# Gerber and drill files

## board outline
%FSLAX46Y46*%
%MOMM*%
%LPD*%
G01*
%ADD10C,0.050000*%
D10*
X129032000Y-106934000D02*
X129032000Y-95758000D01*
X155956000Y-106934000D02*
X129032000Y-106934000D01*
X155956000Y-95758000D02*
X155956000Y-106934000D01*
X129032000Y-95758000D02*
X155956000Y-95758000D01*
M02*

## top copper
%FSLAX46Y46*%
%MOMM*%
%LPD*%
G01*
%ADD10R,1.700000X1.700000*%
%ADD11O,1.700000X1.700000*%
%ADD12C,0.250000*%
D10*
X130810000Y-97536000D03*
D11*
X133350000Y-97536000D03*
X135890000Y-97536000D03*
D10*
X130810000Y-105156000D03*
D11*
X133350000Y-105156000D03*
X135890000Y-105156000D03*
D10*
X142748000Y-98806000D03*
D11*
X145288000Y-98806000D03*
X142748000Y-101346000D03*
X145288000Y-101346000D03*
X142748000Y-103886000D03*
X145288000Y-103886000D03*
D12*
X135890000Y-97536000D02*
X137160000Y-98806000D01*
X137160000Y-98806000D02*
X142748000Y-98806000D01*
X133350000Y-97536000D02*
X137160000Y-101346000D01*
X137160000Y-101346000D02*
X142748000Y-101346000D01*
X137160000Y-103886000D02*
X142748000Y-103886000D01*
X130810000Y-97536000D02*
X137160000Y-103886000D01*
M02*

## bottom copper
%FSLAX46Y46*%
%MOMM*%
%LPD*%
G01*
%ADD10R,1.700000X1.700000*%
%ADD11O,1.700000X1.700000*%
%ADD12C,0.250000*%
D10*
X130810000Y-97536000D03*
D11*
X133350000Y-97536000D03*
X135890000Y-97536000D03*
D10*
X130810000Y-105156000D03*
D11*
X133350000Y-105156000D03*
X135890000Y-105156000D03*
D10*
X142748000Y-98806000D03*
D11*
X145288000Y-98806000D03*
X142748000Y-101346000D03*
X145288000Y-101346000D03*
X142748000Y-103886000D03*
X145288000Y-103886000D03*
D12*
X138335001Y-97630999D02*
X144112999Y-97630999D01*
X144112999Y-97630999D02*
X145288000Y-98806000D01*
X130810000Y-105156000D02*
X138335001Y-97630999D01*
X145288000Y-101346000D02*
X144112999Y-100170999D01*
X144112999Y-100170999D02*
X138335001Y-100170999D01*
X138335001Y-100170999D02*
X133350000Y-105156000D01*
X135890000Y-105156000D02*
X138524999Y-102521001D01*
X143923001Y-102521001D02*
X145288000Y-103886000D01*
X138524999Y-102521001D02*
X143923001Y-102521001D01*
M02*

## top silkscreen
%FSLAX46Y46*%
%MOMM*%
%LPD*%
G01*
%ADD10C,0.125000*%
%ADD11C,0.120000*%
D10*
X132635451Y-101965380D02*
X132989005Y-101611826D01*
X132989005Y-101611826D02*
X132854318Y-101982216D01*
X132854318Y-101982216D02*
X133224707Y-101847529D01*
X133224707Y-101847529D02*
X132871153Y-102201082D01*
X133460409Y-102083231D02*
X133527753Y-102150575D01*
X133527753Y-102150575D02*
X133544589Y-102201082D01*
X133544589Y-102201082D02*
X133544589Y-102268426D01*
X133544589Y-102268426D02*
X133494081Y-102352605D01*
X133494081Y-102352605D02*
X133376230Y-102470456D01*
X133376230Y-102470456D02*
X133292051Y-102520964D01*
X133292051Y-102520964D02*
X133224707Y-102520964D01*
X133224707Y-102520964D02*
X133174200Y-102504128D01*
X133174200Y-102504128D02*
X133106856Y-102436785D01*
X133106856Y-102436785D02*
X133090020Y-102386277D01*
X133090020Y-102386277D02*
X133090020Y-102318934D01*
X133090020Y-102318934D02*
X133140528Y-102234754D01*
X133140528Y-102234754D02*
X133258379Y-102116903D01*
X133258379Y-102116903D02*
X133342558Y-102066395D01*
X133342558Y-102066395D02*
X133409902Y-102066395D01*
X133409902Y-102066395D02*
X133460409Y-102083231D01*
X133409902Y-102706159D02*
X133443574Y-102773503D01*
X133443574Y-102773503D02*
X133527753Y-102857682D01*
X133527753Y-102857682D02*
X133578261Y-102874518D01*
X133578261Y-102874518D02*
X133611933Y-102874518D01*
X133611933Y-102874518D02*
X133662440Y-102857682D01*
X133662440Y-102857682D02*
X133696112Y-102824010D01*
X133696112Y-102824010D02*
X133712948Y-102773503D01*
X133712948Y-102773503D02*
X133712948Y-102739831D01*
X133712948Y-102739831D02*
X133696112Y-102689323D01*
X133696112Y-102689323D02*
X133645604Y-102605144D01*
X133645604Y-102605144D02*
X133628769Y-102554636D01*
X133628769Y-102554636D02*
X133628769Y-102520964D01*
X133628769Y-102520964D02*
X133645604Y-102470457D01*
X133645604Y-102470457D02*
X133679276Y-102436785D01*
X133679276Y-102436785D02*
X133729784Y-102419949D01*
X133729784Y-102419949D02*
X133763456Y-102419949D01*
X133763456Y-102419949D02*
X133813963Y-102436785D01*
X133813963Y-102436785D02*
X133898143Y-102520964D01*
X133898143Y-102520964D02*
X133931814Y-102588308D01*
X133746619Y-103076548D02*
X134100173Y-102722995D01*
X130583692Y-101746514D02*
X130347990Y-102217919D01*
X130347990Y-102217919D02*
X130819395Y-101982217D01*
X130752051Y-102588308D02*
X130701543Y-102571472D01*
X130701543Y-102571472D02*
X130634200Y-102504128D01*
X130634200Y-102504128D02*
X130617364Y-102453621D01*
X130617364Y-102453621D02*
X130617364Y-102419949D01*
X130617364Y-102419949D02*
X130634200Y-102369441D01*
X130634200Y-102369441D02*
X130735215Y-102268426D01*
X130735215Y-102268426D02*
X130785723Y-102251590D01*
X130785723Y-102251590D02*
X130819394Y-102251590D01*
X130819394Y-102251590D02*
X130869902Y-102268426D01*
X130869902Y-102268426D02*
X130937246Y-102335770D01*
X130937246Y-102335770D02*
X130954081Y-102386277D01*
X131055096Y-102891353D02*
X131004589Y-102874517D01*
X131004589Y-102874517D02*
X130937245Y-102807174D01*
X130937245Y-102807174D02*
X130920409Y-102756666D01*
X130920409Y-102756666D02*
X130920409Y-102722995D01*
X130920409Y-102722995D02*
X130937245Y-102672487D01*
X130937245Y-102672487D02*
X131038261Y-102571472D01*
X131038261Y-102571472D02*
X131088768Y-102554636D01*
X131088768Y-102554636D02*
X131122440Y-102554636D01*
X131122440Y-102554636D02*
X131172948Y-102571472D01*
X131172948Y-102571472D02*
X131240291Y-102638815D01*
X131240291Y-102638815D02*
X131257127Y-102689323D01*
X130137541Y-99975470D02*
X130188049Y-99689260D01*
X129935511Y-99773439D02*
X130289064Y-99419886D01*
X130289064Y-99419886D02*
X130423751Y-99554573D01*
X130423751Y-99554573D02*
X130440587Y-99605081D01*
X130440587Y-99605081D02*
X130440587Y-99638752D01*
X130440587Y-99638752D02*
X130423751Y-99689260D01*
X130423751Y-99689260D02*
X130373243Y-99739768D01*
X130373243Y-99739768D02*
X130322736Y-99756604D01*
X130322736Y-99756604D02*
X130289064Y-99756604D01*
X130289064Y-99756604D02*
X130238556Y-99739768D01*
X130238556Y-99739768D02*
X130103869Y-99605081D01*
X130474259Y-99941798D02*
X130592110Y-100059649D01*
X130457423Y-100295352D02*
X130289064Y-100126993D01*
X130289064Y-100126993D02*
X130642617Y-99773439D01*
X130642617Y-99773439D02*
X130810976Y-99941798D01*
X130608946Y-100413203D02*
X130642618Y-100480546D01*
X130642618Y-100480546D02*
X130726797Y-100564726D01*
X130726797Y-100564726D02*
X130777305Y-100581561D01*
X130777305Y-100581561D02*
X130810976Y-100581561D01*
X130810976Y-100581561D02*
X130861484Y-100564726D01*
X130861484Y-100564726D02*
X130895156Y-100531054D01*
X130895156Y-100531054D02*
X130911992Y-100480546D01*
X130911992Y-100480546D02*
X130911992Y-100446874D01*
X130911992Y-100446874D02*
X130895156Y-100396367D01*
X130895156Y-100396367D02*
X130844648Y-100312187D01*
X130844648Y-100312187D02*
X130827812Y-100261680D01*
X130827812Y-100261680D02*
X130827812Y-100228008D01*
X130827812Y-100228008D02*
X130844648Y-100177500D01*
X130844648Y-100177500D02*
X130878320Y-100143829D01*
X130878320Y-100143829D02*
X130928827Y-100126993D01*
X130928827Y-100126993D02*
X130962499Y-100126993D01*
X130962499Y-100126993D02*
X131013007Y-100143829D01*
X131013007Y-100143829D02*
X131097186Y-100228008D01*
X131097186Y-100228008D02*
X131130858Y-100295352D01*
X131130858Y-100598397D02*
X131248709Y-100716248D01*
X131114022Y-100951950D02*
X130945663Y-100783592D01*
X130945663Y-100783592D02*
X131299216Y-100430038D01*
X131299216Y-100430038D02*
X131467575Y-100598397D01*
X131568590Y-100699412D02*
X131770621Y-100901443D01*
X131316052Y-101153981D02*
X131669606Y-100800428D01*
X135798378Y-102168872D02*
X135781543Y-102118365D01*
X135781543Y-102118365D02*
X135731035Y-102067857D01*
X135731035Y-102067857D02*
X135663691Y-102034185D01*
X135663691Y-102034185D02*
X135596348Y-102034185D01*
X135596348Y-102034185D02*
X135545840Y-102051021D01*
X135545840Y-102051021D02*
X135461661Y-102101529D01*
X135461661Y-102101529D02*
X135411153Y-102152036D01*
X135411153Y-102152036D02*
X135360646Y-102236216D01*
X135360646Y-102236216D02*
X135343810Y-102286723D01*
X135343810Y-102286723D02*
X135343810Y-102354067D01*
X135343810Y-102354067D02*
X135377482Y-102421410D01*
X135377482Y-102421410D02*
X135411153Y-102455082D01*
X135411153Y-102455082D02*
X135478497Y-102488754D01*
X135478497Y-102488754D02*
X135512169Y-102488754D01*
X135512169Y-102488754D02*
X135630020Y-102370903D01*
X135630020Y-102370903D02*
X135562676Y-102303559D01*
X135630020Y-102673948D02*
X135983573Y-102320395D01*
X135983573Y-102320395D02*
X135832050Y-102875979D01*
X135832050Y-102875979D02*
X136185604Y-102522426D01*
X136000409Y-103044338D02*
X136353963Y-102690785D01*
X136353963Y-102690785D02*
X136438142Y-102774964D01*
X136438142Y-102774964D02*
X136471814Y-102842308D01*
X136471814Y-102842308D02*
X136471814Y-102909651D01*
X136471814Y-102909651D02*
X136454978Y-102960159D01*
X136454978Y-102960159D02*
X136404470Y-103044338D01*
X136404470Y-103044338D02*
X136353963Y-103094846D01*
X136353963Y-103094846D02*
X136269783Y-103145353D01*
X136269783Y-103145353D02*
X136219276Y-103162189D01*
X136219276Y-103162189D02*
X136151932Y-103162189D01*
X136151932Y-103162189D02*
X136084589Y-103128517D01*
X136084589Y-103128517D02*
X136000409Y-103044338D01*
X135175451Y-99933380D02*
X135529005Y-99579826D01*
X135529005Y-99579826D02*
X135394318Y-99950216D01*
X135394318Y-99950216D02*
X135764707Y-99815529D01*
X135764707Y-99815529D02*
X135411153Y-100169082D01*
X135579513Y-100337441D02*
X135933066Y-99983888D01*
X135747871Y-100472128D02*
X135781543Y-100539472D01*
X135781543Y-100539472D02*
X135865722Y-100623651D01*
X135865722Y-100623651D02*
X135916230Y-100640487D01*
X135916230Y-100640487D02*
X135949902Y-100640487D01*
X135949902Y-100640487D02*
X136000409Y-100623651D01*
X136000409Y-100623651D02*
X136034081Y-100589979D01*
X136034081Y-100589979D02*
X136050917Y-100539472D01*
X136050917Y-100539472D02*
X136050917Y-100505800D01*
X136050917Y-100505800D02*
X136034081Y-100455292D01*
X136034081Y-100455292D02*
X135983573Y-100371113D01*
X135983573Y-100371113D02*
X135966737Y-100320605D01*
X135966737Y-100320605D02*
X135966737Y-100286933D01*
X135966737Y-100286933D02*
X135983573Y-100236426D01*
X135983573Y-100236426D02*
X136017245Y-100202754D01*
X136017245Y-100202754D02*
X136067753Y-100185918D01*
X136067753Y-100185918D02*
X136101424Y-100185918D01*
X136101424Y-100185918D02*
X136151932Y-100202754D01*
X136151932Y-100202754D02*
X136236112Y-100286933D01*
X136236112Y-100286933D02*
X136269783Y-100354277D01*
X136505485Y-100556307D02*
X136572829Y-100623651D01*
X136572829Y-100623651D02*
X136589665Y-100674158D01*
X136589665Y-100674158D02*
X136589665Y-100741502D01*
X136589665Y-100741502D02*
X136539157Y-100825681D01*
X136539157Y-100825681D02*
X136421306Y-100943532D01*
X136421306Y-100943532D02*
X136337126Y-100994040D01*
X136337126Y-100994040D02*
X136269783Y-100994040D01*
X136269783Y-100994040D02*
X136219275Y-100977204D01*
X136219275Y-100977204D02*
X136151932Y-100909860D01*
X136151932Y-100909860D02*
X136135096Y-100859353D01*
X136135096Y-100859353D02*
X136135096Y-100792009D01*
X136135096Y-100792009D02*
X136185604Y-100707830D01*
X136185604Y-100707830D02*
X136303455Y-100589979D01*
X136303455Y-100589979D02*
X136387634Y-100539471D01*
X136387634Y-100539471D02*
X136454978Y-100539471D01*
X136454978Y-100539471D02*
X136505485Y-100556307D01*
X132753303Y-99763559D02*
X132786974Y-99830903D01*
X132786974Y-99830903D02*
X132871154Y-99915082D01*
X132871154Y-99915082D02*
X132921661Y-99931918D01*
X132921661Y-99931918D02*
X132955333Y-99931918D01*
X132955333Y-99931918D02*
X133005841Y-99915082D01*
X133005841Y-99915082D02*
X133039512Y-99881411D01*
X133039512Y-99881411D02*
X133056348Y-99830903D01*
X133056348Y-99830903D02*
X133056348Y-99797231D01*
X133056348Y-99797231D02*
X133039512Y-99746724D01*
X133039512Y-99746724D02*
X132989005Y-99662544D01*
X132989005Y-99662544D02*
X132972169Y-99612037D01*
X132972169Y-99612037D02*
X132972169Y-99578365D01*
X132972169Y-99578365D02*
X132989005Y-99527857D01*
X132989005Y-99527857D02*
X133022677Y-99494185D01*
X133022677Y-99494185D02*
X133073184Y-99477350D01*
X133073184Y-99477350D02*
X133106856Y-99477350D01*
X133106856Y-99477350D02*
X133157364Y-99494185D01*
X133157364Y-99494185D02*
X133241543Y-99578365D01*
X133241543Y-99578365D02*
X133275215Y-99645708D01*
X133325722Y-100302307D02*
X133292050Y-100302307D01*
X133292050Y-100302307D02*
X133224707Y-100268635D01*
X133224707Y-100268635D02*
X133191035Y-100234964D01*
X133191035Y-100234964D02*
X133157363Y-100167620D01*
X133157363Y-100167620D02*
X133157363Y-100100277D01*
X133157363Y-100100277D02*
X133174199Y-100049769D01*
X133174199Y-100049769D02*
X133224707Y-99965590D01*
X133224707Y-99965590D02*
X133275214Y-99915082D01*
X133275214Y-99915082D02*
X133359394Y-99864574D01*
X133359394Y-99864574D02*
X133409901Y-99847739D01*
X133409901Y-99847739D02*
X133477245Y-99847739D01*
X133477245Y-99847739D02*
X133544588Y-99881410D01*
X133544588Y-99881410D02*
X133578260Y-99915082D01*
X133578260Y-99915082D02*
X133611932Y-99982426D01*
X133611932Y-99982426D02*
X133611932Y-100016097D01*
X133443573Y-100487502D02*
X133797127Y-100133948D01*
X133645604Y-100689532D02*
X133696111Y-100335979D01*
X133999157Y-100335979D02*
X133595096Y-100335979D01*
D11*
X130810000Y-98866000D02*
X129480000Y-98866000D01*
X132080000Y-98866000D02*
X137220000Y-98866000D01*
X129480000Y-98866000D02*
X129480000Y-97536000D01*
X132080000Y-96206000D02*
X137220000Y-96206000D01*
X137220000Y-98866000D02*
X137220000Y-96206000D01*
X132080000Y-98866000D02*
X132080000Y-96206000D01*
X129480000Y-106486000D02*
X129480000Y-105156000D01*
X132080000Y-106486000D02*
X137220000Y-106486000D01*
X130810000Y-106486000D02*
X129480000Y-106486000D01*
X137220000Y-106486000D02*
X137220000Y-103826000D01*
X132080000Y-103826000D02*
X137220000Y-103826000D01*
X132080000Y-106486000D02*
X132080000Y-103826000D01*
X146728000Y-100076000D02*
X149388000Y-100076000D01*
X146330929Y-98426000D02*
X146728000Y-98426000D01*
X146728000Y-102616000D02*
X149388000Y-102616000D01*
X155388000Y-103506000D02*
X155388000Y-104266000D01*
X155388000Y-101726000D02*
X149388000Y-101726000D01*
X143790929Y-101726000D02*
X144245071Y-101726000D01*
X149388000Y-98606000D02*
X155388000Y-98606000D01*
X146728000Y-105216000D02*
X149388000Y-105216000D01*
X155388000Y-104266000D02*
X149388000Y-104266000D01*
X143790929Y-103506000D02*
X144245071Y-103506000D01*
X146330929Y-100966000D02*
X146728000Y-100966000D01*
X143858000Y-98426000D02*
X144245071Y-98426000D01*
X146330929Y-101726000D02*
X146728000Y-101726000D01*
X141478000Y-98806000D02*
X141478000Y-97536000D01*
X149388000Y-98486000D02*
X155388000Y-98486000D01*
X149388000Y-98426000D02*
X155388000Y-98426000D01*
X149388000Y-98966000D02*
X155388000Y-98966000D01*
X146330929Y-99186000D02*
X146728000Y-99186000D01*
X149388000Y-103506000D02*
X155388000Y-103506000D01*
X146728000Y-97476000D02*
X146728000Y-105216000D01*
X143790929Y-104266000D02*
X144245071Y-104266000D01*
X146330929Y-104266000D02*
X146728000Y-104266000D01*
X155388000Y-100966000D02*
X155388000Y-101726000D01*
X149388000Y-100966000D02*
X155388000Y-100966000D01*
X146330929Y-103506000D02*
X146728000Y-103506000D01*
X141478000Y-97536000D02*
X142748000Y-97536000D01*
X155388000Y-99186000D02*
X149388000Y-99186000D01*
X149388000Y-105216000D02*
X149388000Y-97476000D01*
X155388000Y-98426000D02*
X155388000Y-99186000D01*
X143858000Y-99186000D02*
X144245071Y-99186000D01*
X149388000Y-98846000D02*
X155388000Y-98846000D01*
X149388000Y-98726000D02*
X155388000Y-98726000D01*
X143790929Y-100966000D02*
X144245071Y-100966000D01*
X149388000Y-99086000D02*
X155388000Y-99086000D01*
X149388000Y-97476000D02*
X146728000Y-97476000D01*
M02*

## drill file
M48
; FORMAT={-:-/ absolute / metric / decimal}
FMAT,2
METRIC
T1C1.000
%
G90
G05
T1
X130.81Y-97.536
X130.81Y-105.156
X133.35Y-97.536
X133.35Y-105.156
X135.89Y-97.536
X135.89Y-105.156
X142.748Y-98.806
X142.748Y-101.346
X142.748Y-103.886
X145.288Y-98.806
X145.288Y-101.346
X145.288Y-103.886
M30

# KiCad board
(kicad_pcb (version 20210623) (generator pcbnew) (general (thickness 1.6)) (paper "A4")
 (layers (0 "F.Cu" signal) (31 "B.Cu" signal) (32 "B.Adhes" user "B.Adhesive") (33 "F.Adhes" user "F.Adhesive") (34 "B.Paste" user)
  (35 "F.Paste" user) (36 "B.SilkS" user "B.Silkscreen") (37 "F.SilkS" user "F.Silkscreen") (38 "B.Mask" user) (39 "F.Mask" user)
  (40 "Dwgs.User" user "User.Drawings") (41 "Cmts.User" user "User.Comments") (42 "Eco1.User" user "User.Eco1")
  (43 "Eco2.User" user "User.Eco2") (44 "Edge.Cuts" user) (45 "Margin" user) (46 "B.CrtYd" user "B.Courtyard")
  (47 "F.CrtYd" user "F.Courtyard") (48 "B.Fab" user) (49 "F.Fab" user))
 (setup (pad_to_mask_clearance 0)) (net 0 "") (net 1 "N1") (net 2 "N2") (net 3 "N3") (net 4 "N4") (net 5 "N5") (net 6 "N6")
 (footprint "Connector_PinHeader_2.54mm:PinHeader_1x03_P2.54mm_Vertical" (layer "F.Cu") (at 130.81 97.536 90)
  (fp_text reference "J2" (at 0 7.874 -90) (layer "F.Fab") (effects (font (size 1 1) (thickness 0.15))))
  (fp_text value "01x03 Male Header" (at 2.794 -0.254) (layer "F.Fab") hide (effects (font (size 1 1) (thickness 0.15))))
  (fp_line (start -1.33 0) (end -1.33 -1.33) (layer "F.SilkS") (width 0.12))
  (fp_line (start -1.33 1.27) (end -1.33 6.41) (layer "F.SilkS") (width 0.12))
  (fp_line (start -1.33 -1.33) (end 0 -1.33) (layer "F.SilkS") (width 0.12))
  (fp_line (start 1.33 1.27) (end 1.33 6.41) (layer "F.SilkS") (width 0.12))
  (fp_line (start -1.33 6.41) (end 1.33 6.41) (layer "F.SilkS") (width 0.12))
  (fp_line (start -1.33 1.27) (end 1.33 1.27) (layer "F.SilkS") (width 0.12))
  (pad "1" thru_hole rect locked (at 0 0 90) (size 1.7 1.7) (drill 1) (layers *.Cu *.Mask) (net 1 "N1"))
  (pad "2" thru_hole oval locked (at 0 2.54 90) (size 1.7 1.7) (drill 1) (layers *.Cu *.Mask) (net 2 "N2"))
  (pad "3" thru_hole oval locked (at 0 5.08 90) (size 1.7 1.7) (drill 1) (layers *.Cu *.Mask) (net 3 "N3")))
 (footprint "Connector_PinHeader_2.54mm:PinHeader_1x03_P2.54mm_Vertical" (layer "F.Cu") (at 130.81 105.156 90)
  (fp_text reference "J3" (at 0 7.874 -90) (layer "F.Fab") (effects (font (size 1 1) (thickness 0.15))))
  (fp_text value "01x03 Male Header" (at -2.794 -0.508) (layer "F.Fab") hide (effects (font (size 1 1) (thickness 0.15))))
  (fp_line (start -1.33 -1.33) (end 0 -1.33) (layer "F.SilkS") (width 0.12))
  (fp_line (start -1.33 1.27) (end -1.33 6.41) (layer "F.SilkS") (width 0.12))
  (fp_line (start -1.33 0) (end -1.33 -1.33) (layer "F.SilkS") (width 0.12))
  (fp_line (start -1.33 6.41) (end 1.33 6.41) (layer "F.SilkS") (width 0.12))
  (fp_line (start 1.33 1.27) (end 1.33 6.41) (layer "F.SilkS") (width 0.12))
  (fp_line (start -1.33 1.27) (end 1.33 1.27) (layer "F.SilkS") (width 0.12))
  (pad "1" thru_hole rect locked (at 0 0 90) (size 1.7 1.7) (drill 1) (layers *.Cu *.Mask) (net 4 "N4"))
  (pad "2" thru_hole oval locked (at 0 2.54 90) (size 1.7 1.7) (drill 1) (layers *.Cu *.Mask) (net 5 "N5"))
  (pad "3" thru_hole oval locked (at 0 5.08 90) (size 1.7 1.7) (drill 1) (layers *.Cu *.Mask) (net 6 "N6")))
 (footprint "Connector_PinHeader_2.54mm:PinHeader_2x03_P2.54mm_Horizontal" (layer "F.Cu") (at 142.748 98.806)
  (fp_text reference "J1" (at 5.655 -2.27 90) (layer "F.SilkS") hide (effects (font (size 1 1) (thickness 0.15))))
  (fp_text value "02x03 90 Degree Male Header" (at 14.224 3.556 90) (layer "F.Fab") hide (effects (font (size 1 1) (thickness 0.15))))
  (fp_line (start 3.98 1.27) (end 6.64 1.27) (layer "F.SilkS") (width 0.12))
  (fp_line (start 3.582929 -0.38) (end 3.98 -0.38) (layer "F.SilkS") (width 0.12))
  (fp_line (start 3.98 3.81) (end 6.64 3.81) (layer "F.SilkS") (width 0.12))
  (fp_line (start 12.64 4.7) (end 12.64 5.46) (layer "F.SilkS") (width 0.12))
  (fp_line (start 12.64 2.92) (end 6.64 2.92) (layer "F.SilkS") (width 0.12))
  (fp_line (start 1.042929 2.92) (end 1.497071 2.92) (layer "F.SilkS") (width 0.12))
  (fp_line (start 6.64 -0.2) (end 12.64 -0.2) (layer "F.SilkS") (width 0.12))
  (fp_line (start 3.98 6.41) (end 6.64 6.41) (layer "F.SilkS") (width 0.12))
  (fp_line (start 12.64 5.46) (end 6.64 5.46) (layer "F.SilkS") (width 0.12))
  (fp_line (start 1.042929 4.7) (end 1.497071 4.7) (layer "F.SilkS") (width 0.12))
  (fp_line (start 3.582929 2.16) (end 3.98 2.16) (layer "F.SilkS") (width 0.12))
  (fp_line (start 1.11 -0.38) (end 1.497071 -0.38) (layer "F.SilkS") (width 0.12))
  (fp_line (start 3.582929 2.92) (end 3.98 2.92) (layer "F.SilkS") (width 0.12))
  (fp_line (start -1.27 0) (end -1.27 -1.27) (layer "F.SilkS") (width 0.12))
  (fp_line (start 6.64 -0.32) (end 12.64 -0.32) (layer "F.SilkS") (width 0.12))
  (fp_line (start 6.64 -0.38) (end 12.64 -0.38) (layer "F.SilkS") (width 0.12))
  (fp_line (start 6.64 0.16) (end 12.64 0.16) (layer "F.SilkS") (width 0.12))
  (fp_line (start 3.582929 0.38) (end 3.98 0.38) (layer "F.SilkS") (width 0.12))
  (fp_line (start 6.64 4.7) (end 12.64 4.7) (layer "F.SilkS") (width 0.12))
  (fp_line (start 3.98 -1.33) (end 3.98 6.41) (layer "F.SilkS") (width 0.12))
  (fp_line (start 1.042929 5.46) (end 1.497071 5.46) (layer "F.SilkS") (width 0.12))
  (fp_line (start 3.582929 5.46) (end 3.98 5.46) (layer "F.SilkS") (width 0.12))
  (fp_line (start 12.64 2.16) (end 12.64 2.92) (layer "F.SilkS") (width 0.12))
  (fp_line (start 6.64 2.16) (end 12.64 2.16) (layer "F.SilkS") (width 0.12))
  (fp_line (start 3.582929 4.7) (end 3.98 4.7) (layer "F.SilkS") (width 0.12))
  (fp_line (start -1.27 -1.27) (end 0 -1.27) (layer "F.SilkS") (width 0.12))
  (fp_line (start 12.64 0.38) (end 6.64 0.38) (layer "F.SilkS") (width 0.12))
  (fp_line (start 6.64 6.41) (end 6.64 -1.33) (layer "F.SilkS") (width 0.12))
  (fp_line (start 12.64 -0.38) (end 12.64 0.38) (layer "F.SilkS") (width 0.12))
  (fp_line (start 1.11 0.38) (end 1.497071 0.38) (layer "F.SilkS") (width 0.12))
  (fp_line (start 6.64 0.04) (end 12.64 0.04) (layer "F.SilkS") (width 0.12))
  (fp_line (start 6.64 -0.08) (end 12.64 -0.08) (layer "F.SilkS") (width 0.12))
  (fp_line (start 1.042929 2.16) (end 1.497071 2.16) (layer "F.SilkS") (width 0.12))
  (fp_line (start 6.64 0.28) (end 12.64 0.28) (layer "F.SilkS") (width 0.12))
  (fp_line (start 6.64 -1.33) (end 3.98 -1.33) (layer "F.SilkS") (width 0.12))
  (pad "1" thru_hole rect locked (at 0 0) (size 1.7 1.7) (drill 1) (layers *.Cu *.Mask) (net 3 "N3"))
  (pad "2" thru_hole oval locked (at 2.54 0) (size 1.7 1.7) (drill 1) (layers *.Cu *.Mask) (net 4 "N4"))
  (pad "3" thru_hole oval locked (at 0 2.54) (size 1.7 1.7) (drill 1) (layers *.Cu *.Mask) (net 2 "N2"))
  (pad "4" thru_hole oval locked (at 2.54 2.54) (size 1.7 1.7) (drill 1) (layers *.Cu *.Mask) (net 5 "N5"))
  (pad "5" thru_hole oval locked (at 0 5.08) (size 1.7 1.7) (drill 1) (layers *.Cu *.Mask) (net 1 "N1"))
  (pad "6" thru_hole oval locked (at 2.54 5.08) (size 1.7 1.7) (drill 1) (layers *.Cu *.Mask) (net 6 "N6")))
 (gr_line (start 129.032 106.934) (end 129.032 95.758) (layer "Edge.Cuts") (width 0.05))
 (gr_line (start 155.956 106.934) (end 129.032 106.934) (layer "Edge.Cuts") (width 0.05))
 (gr_line (start 155.956 95.758) (end 155.956 106.934) (layer "Edge.Cuts") (width 0.05))
 (gr_line (start 129.032 95.758) (end 155.956 95.758) (layer "Edge.Cuts") (width 0.05))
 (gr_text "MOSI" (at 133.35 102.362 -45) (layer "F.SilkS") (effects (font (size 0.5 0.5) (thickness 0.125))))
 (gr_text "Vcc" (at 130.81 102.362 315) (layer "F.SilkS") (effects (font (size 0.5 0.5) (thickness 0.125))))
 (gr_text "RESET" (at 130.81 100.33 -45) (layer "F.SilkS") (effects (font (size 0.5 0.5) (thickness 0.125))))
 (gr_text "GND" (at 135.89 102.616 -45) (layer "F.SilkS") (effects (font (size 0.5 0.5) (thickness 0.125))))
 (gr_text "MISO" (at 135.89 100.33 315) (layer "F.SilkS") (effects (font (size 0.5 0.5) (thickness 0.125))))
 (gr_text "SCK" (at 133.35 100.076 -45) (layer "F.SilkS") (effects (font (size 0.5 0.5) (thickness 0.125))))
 (segment (start 135.89 97.536) (end 137.16 98.806) (width 0.25) (layer "F.Cu") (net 3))
 (segment (start 137.16 98.806) (end 142.748 98.806) (width 0.25) (layer "F.Cu") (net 3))
 (segment (start 138.335001 97.630999) (end 144.112999 97.630999) (width 0.25) (layer "B.Cu") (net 4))
 (segment (start 144.112999 97.630999) (end 145.288 98.806) (width 0.25) (layer "B.Cu") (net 4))
 (segment (start 130.81 105.156) (end 138.335001 97.630999) (width 0.25) (layer "B.Cu") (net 4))
 (segment (start 133.35 97.536) (end 137.16 101.346) (width 0.25) (layer "F.Cu") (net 2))
 (segment (start 137.16 101.346) (end 142.748 101.346) (width 0.25) (layer "F.Cu") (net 2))
 (segment (start 145.288 101.346) (end 144.112999 100.170999) (width 0.25) (layer "B.Cu") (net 5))
 (segment (start 144.112999 100.170999) (end 138.335001 100.170999) (width 0.25) (layer "B.Cu") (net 5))
 (segment (start 138.335001 100.170999) (end 133.35 105.156) (width 0.25) (layer "B.Cu") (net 5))
 (segment (start 137.16 103.886) (end 142.748 103.886) (width 0.25) (layer "F.Cu") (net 1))
 (segment (start 130.81 97.536) (end 137.16 103.886) (width 0.25) (layer "F.Cu") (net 1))
 (segment (start 135.89 105.156) (end 138.524999 102.521001) (width 0.25) (layer "B.Cu") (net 6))
 (segment (start 143.923001 102.521001) (end 145.288 103.886) (width 0.25) (layer "B.Cu") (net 6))
 (segment (start 138.524999 102.521001) (end 143.923001 102.521001) (width 0.25) (layer "B.Cu") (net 6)))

